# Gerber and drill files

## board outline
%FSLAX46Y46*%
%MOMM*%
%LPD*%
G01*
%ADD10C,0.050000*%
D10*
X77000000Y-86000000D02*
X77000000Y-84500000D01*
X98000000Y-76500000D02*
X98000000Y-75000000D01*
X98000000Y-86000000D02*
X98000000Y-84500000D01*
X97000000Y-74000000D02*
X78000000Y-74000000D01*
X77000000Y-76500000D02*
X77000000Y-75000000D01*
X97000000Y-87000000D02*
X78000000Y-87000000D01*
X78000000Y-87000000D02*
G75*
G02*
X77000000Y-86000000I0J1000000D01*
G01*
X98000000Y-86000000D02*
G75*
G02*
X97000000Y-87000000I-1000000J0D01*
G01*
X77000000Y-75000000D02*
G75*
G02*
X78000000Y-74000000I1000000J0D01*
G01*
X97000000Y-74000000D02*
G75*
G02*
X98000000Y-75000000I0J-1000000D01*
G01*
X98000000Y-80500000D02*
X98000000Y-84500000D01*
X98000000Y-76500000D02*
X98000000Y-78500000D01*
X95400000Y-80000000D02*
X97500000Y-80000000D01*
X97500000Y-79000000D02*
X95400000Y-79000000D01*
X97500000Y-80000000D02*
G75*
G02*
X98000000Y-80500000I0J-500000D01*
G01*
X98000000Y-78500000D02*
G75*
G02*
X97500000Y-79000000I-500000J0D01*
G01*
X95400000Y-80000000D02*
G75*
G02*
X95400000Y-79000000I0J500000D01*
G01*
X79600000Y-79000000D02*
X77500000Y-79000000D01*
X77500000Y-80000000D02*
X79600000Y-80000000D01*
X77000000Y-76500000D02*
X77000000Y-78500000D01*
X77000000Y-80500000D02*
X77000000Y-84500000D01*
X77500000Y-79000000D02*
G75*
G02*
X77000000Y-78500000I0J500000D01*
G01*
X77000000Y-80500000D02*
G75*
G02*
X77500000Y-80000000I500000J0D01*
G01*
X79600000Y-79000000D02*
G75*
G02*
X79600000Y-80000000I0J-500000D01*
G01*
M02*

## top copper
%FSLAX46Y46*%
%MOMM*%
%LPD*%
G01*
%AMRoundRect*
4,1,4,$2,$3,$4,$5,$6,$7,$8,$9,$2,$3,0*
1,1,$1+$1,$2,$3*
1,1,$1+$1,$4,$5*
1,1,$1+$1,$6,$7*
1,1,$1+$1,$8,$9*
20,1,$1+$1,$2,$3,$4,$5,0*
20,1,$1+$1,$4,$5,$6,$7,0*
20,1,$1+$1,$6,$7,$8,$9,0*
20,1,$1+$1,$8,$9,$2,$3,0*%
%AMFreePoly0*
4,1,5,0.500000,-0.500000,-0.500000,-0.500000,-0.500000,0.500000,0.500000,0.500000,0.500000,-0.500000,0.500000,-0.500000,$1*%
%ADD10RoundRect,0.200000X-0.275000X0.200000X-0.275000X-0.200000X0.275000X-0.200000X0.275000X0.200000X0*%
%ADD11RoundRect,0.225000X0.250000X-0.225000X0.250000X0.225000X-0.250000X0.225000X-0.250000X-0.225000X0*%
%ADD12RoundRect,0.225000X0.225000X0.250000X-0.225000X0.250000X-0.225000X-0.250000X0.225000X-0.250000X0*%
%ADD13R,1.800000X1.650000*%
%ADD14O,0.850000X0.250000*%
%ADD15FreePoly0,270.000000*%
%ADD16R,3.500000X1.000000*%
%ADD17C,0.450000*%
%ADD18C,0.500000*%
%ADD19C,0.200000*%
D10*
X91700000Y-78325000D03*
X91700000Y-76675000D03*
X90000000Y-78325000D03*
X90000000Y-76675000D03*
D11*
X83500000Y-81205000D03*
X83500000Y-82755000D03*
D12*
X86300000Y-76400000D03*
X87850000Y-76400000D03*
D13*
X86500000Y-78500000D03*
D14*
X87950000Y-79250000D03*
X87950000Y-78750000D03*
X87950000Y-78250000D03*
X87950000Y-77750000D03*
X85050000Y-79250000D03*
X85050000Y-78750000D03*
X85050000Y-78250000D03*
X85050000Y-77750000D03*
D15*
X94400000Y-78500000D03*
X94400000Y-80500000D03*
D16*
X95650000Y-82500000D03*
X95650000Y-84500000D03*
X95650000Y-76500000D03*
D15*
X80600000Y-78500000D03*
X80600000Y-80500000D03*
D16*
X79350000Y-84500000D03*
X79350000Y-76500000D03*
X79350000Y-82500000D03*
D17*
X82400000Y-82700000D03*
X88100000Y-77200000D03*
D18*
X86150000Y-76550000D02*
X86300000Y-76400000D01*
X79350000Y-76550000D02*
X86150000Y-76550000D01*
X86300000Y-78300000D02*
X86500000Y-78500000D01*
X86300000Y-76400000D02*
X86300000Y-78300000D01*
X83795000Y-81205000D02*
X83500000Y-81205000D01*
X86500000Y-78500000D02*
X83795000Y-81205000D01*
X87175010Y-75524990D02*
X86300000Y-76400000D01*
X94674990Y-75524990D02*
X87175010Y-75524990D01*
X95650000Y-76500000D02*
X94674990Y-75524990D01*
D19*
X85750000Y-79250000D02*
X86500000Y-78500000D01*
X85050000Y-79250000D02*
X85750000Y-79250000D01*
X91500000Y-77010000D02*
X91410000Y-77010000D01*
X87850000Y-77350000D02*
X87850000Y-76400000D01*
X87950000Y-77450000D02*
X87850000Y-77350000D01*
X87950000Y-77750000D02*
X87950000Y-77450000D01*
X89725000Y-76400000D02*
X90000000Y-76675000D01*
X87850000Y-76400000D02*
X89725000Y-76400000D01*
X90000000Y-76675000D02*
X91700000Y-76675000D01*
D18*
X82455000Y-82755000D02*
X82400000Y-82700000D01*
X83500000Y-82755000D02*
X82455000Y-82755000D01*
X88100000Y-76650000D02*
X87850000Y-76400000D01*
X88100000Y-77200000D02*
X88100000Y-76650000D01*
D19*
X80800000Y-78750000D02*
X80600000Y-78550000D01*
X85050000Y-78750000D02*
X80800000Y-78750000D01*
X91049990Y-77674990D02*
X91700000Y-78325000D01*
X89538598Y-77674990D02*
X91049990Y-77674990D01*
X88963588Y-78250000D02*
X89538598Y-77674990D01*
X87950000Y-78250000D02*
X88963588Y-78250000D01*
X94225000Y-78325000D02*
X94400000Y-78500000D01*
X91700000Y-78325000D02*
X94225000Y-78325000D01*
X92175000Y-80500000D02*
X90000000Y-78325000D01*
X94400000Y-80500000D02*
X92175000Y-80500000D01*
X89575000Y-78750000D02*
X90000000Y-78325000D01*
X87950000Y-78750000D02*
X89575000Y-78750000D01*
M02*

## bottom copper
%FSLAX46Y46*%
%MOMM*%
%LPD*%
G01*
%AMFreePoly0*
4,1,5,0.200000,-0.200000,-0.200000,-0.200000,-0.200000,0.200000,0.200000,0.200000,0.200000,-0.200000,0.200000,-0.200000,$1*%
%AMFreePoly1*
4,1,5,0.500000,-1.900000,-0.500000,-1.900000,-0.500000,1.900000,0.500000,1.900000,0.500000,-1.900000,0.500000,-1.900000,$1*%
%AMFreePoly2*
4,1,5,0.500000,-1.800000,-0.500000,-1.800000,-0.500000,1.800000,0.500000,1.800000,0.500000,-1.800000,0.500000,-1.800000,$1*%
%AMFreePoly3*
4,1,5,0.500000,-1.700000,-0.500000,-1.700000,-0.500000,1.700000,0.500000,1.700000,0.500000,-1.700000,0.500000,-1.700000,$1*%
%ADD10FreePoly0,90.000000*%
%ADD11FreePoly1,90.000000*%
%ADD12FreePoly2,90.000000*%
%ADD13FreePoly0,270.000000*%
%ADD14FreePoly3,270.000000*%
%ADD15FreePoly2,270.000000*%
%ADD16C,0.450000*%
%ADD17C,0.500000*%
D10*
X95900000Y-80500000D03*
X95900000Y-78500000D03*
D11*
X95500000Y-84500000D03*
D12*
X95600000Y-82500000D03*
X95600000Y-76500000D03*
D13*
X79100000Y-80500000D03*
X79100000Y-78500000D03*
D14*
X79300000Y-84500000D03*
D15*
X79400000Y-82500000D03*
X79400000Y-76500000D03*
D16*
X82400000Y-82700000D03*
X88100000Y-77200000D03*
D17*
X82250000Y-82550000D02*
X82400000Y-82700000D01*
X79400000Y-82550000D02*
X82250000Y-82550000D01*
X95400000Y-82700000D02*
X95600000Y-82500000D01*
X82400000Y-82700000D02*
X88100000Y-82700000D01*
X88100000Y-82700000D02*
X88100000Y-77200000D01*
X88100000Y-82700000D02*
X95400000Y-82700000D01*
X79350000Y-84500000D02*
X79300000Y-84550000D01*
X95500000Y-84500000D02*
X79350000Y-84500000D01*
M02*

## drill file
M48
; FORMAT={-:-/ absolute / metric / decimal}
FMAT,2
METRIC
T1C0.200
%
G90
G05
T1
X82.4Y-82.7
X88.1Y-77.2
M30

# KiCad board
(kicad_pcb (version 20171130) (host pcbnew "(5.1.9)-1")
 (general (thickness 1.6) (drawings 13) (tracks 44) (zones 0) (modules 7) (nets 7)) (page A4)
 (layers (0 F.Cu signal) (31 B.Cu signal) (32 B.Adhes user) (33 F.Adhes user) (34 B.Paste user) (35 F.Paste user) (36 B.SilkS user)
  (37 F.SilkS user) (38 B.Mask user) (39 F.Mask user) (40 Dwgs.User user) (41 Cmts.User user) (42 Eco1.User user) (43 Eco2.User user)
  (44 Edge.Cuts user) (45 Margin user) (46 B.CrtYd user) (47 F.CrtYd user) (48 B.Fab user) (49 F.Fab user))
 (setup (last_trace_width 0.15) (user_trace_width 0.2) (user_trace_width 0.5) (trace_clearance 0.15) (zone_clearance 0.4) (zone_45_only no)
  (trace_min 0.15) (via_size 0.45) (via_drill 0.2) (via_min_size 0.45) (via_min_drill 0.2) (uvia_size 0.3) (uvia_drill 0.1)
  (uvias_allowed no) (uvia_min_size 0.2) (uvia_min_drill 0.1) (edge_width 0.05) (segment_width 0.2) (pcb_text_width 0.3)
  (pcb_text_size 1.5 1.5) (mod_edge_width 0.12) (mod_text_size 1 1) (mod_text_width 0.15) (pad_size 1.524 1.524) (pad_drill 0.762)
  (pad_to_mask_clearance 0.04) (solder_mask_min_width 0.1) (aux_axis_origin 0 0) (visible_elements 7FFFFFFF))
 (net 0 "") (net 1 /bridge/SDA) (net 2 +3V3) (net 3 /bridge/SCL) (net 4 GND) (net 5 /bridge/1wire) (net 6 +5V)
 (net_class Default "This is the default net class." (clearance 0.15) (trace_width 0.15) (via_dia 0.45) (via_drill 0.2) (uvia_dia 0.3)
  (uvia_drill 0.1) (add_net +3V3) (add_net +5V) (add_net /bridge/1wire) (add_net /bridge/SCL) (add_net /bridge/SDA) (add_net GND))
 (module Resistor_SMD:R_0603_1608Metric (layer F.Cu) (at 91.7 77.5 270)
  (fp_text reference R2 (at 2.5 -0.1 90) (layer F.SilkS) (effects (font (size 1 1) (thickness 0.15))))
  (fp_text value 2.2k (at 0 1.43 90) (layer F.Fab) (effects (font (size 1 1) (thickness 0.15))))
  (pad 2 smd roundrect (at 0.825 0 270) (size 0.8 0.95) (layers F.Cu F.Paste F.Mask) (roundrect_rratio 0.25) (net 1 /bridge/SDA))
  (pad 1 smd roundrect (at -0.825 0 270) (size 0.8 0.95) (layers F.Cu F.Paste F.Mask) (roundrect_rratio 0.25) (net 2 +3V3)))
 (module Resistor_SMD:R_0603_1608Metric (layer F.Cu) (at 90 77.5 270)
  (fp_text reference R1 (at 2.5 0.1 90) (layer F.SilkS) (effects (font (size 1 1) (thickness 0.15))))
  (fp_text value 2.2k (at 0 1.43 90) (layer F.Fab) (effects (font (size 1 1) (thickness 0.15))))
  (pad 2 smd roundrect (at 0.825 0 270) (size 0.8 0.95) (layers F.Cu F.Paste F.Mask) (roundrect_rratio 0.25) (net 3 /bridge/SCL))
  (pad 1 smd roundrect (at -0.825 0 270) (size 0.8 0.95) (layers F.Cu F.Paste F.Mask) (roundrect_rratio 0.25) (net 2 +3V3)))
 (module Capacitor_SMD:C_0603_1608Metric (layer F.Cu) (at 83.5 81.98 90)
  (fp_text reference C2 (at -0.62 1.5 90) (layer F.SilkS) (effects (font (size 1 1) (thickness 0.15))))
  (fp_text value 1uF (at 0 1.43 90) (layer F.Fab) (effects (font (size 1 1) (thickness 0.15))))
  (pad 2 smd roundrect (at 0.775 0 90) (size 0.9 0.95) (layers F.Cu F.Paste F.Mask) (roundrect_rratio 0.25) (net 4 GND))
  (pad 1 smd roundrect (at -0.775 0 90) (size 0.9 0.95) (layers F.Cu F.Paste F.Mask) (roundrect_rratio 0.25) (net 2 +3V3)))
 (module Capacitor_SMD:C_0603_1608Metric (layer F.Cu) (at 87.075 76.4 180)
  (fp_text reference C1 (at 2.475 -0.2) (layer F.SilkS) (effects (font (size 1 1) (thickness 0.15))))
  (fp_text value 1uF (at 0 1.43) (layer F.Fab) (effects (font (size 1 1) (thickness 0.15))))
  (pad 2 smd roundrect (at 0.775 0 180) (size 0.9 0.95) (layers F.Cu F.Paste F.Mask) (roundrect_rratio 0.25) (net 4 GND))
  (pad 1 smd roundrect (at -0.775 0 180) (size 0.9 0.95) (layers F.Cu F.Paste F.Mask) (roundrect_rratio 0.25) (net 2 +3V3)))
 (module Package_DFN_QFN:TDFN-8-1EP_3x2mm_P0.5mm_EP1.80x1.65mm (layer F.Cu) (at 86.5 78.5)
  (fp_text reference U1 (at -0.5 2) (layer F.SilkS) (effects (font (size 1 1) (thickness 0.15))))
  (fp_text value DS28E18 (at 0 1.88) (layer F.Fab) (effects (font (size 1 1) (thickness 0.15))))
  (pad "" smd rect (at 0 0.5) (size 0.7 0.65) (layers F.Paste))
  (pad "" smd rect (at 0 -0.5) (size 0.7 0.65) (layers F.Paste)) (pad "" smd rect (at 0 0) (size 1.8 0.7) (layers F.Paste))
  (pad 9 smd rect (at 0 0) (size 1.8 1.65) (layers F.Cu F.Mask) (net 4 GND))
  (pad 5 smd oval (at 1.45 0.75) (size 0.85 0.25) (layers F.Cu F.Paste F.Mask))
  (pad 6 smd oval (at 1.45 0.25) (size 0.85 0.25) (layers F.Cu F.Paste F.Mask) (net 3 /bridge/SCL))
  (pad 7 smd oval (at 1.45 -0.25) (size 0.85 0.25) (layers F.Cu F.Paste F.Mask) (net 1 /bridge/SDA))
  (pad 8 smd oval (at 1.45 -0.75) (size 0.85 0.25) (layers F.Cu F.Paste F.Mask) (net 2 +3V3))
  (pad 4 smd oval (at -1.45 0.75) (size 0.85 0.25) (layers F.Cu F.Paste F.Mask) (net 4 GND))
  (pad 3 smd oval (at -1.45 0.25) (size 0.85 0.25) (layers F.Cu F.Paste F.Mask) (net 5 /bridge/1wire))
  (pad 2 smd oval (at -1.45 -0.25) (size 0.85 0.25) (layers F.Cu F.Paste F.Mask))
  (pad 1 smd oval (at -1.45 -0.75) (size 0.85 0.25) (layers F.Cu F.Paste F.Mask)))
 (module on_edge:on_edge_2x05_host (layer F.Cu) (at 98 80.5 270)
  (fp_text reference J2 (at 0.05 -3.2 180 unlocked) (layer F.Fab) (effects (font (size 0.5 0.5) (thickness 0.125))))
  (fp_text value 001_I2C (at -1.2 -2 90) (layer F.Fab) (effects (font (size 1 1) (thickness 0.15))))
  (fp_line (start 0 0) (end 4 0) (layer Edge.Cuts) (width 0.05))
  (fp_line (start -4 0) (end -2 0) (layer Edge.Cuts) (width 0.05))
  (fp_line (start -0.5 2.6) (end -0.5 0.5) (layer Edge.Cuts) (width 0.05))
  (fp_line (start -1.5 0.5) (end -1.5 2.6) (layer Edge.Cuts) (width 0.05))
  (fp_arc (start 0 0.5) (end 0 0) (angle -90) (layer Edge.Cuts) (width 0.05))
  (fp_arc (start -2 0.5) (end -1.5 0.5) (angle -90) (layer Edge.Cuts) (width 0.05))
  (fp_arc (start -1 2.6) (end -1.5 2.6) (angle -180) (layer Edge.Cuts) (width 0.05))
  (pad 2 smd custom (at -2 3.6 270) (size 1 1) (layers F.Cu F.Mask) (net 1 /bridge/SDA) (zone_connect 0)
   (options (clearance outline) (anchor rect)) (primitives))
  (pad 3 smd custom (at 0 3.6 270) (size 1 1) (layers F.Cu F.Mask) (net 3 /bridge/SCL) (zone_connect 0)
   (options (clearance outline) (anchor rect)) (primitives))
  (pad 8 smd custom (at 0 2.1 90) (size 0.4 0.4) (layers B.Cu B.Mask) (zone_connect 0) (options (clearance outline) (anchor rect))
   (primitives))
  (pad 7 smd custom (at -2 2.1 90) (size 0.4 0.4) (layers B.Cu B.Mask) (zone_connect 0) (options (clearance outline) (anchor rect))
   (primitives))
  (pad 4 smd rect (at 2 2.35 270) (size 1 3.5) (layers F.Cu F.Mask) (zone_connect 0))
  (pad 10 smd custom (at 4 2.5 90) (size 1 3.8) (layers B.Cu B.Mask) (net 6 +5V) (zone_connect 0)
   (options (clearance outline) (anchor rect)) (primitives))
  (pad 9 smd custom (at 2 2.4 90) (size 1 3.6) (layers B.Cu B.Mask) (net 2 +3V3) (zone_connect 0)
   (options (clearance outline) (anchor rect)) (primitives))
  (pad 6 smd custom (at -4 2.4 90) (size 1 3.6) (layers B.Cu B.Mask) (zone_connect 0) (options (clearance outline) (anchor rect))
   (primitives))
  (pad 5 smd rect (at 4 2.35 270) (size 1 3.5) (layers F.Cu F.Mask) (zone_connect 0))
  (pad 1 smd rect (at -4 2.35 270) (size 1 3.5) (layers F.Cu F.Mask) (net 4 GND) (zone_connect 0)))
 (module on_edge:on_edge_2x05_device (layer F.Cu) (at 77 80.5 270)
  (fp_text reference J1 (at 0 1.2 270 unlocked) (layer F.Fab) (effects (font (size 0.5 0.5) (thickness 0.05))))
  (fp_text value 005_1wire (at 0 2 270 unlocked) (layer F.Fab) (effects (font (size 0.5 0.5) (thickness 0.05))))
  (fp_line (start -1.5 -2.6) (end -1.5 -0.5) (layer Edge.Cuts) (width 0.05))
  (fp_line (start -0.5 -0.5) (end -0.5 -2.6) (layer Edge.Cuts) (width 0.05))
  (fp_line (start -4 0) (end -2 0) (layer Edge.Cuts) (width 0.05))
  (fp_line (start 0 0) (end 4 0) (layer Edge.Cuts) (width 0.05))
  (fp_arc (start -2 -0.5) (end -2 0) (angle -90) (layer Edge.Cuts) (width 0.05))
  (fp_arc (start 0 -0.5) (end -0.5 -0.5) (angle -90) (layer Edge.Cuts) (width 0.05))
  (fp_arc (start -1 -2.6) (end -0.5 -2.6) (angle -180) (layer Edge.Cuts) (width 0.05))
  (pad 2 smd custom (at -2 -3.6 270) (size 1 1) (layers F.Cu F.Mask) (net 5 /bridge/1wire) (zone_connect 0)
   (options (clearance outline) (anchor rect)) (primitives))
  (pad 3 smd custom (at 0 -3.6 270) (size 1 1) (layers F.Cu F.Mask) (zone_connect 0) (options (clearance outline) (anchor rect))
   (primitives))
  (pad 8 smd custom (at 0 -2.1 270) (size 0.4 0.4) (layers B.Cu B.Mask) (zone_connect 0) (options (clearance outline) (anchor rect))
   (primitives))
  (pad 7 smd custom (at -2 -2.1 270) (size 0.4 0.4) (layers B.Cu B.Mask) (zone_connect 0) (options (clearance outline) (anchor rect))
   (primitives))
  (pad 10 smd custom (at 4 -2.3 270) (size 1 3.4) (layers B.Cu B.Mask) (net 6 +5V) (zone_connect 0)
   (options (clearance outline) (anchor rect)) (primitives))
  (pad 9 smd custom (at 2 -2.4 270) (size 1 3.6) (layers B.Cu B.Mask) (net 2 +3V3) (zone_connect 0)
   (options (clearance outline) (anchor rect)) (primitives))
  (pad 6 smd custom (at -4 -2.4 270) (size 1 3.6) (layers B.Cu B.Mask) (zone_connect 0) (options (clearance outline) (anchor rect))
   (primitives))
  (pad 5 smd rect (at 4 -2.35 90) (size 1 3.5) (layers F.Cu F.Mask) (zone_connect 0))
  (pad 1 smd rect (at -4 -2.35 90) (size 1 3.5) (layers F.Cu F.Mask) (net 4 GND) (zone_connect 0))
  (pad 4 smd rect (at 2 -2.35 90) (size 1 3.5) (layers F.Cu F.Mask) (zone_connect 0)))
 (gr_line (start 77 86) (end 77 84.5) (layer Edge.Cuts) (width 0.05))
 (gr_line (start 98 76.5) (end 98 75) (layer Edge.Cuts) (width 0.05))
 (gr_line (start 98 86) (end 98 84.5) (layer Edge.Cuts) (width 0.05))
 (gr_line (start 97 74) (end 78 74) (layer Edge.Cuts) (width 0.05))
 (gr_line (start 77 76.5) (end 77 75) (layer Edge.Cuts) (width 0.05))
 (gr_line (start 97 87) (end 78 87) (layer Edge.Cuts) (width 0.05))
 (gr_arc (start 78 86) (end 77 86) (angle -90) (layer Edge.Cuts) (width 0.05))
 (gr_arc (start 97 86) (end 97 87) (angle -90) (layer Edge.Cuts) (width 0.05))
 (gr_arc (start 78 75) (end 78 74) (angle -90) (layer Edge.Cuts) (width 0.05))
 (gr_arc (start 97 75) (end 98 75) (angle -90) (layer Edge.Cuts) (width 0.05))
 (segment (start 86.15 76.55) (end 86.3 76.4) (width 0.5) (layer F.Cu) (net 4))
 (segment (start 79.35 76.55) (end 86.15 76.55) (width 0.5) (layer F.Cu) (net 4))
 (segment (start 86.3 78.3) (end 86.5 78.5) (width 0.5) (layer F.Cu) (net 4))
 (segment (start 86.3 76.4) (end 86.3 78.3) (width 0.5) (layer F.Cu) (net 4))
 (segment (start 83.795 81.205) (end 83.5 81.205) (width 0.5) (layer F.Cu) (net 4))
 (segment (start 86.5 78.5) (end 83.795 81.205) (width 0.5) (layer F.Cu) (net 4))
 (segment (start 87.17501 75.52499) (end 86.3 76.4) (width 0.5) (layer F.Cu) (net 4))
 (segment (start 94.67499 75.52499) (end 87.17501 75.52499) (width 0.5) (layer F.Cu) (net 4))
 (segment (start 95.65 76.5) (end 94.67499 75.52499) (width 0.5) (layer F.Cu) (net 4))
 (segment (start 85.75 79.25) (end 86.5 78.5) (width 0.2) (layer F.Cu) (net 4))
 (segment (start 85.05 79.25) (end 85.75 79.25) (width 0.2) (layer F.Cu) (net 4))
 (segment (start 82.25 82.55) (end 82.4 82.7) (width 0.5) (layer B.Cu) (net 2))
 (via (at 82.4 82.7) (size 0.45) (drill 0.2) (layers F.Cu B.Cu) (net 2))
 (segment (start 79.4 82.55) (end 82.25 82.55) (width 0.5) (layer B.Cu) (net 2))
 (segment (start 91.5 77.01) (end 91.41 77.01) (width 0.2) (layer F.Cu) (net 2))
 (segment (start 87.85 77.35) (end 87.85 76.4) (width 0.2) (layer F.Cu) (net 2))
 (segment (start 87.95 77.45) (end 87.85 77.35) (width 0.2) (layer F.Cu) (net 2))
 (segment (start 87.95 77.75) (end 87.95 77.45) (width 0.2) (layer F.Cu) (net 2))
 (segment (start 89.725 76.4) (end 90 76.675) (width 0.2) (layer F.Cu) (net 2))
 (segment (start 87.85 76.4) (end 89.725 76.4) (width 0.2) (layer F.Cu) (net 2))
 (segment (start 90 76.675) (end 91.7 76.675) (width 0.2) (layer F.Cu) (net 2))
 (segment (start 82.455 82.755) (end 82.4 82.7) (width 0.5) (layer F.Cu) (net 2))
 (segment (start 83.5 82.755) (end 82.455 82.755) (width 0.5) (layer F.Cu) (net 2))
 (segment (start 95.4 82.7) (end 95.6 82.5) (width 0.5) (layer B.Cu) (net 2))
 (via (at 88.1 77.2) (size 0.45) (drill 0.2) (layers F.Cu B.Cu) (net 2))
 (segment (start 82.4 82.7) (end 88.1 82.7) (width 0.5) (layer B.Cu) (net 2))
 (segment (start 88.1 82.7) (end 88.1 77.2) (width 0.5) (layer B.Cu) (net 2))
 (segment (start 88.1 82.7) (end 95.4 82.7) (width 0.5) (layer B.Cu) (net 2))
 (segment (start 88.1 76.65) (end 87.85 76.4) (width 0.5) (layer F.Cu) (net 2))
 (segment (start 88.1 77.2) (end 88.1 76.65) (width 0.5) (layer F.Cu) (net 2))
 (segment (start 80.8 78.75) (end 80.6 78.55) (width 0.2) (layer F.Cu) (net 5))
 (segment (start 85.05 78.75) (end 80.8 78.75) (width 0.2) (layer F.Cu) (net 5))
 (segment (start 79.35 84.5) (end 79.3 84.55) (width 0.5) (layer B.Cu) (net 6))
 (segment (start 95.5 84.5) (end 79.35 84.5) (width 0.5) (layer B.Cu) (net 6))
 (segment (start 91.04999 77.67499) (end 91.7 78.325) (width 0.2) (layer F.Cu) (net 1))
 (segment (start 89.538598 77.67499) (end 91.04999 77.67499) (width 0.2) (layer F.Cu) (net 1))
 (segment (start 88.963588 78.25) (end 89.538598 77.67499) (width 0.2) (layer F.Cu) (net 1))
 (segment (start 87.95 78.25) (end 88.963588 78.25) (width 0.2) (layer F.Cu) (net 1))
 (segment (start 94.225 78.325) (end 94.4 78.5) (width 0.2) (layer F.Cu) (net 1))
 (segment (start 91.7 78.325) (end 94.225 78.325) (width 0.2) (layer F.Cu) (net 1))
 (segment (start 92.175 80.5) (end 90 78.325) (width 0.2) (layer F.Cu) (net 3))
 (segment (start 94.4 80.5) (end 92.175 80.5) (width 0.2) (layer F.Cu) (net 3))
 (segment (start 89.575 78.75) (end 90 78.325) (width 0.2) (layer F.Cu) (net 3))
 (segment (start 87.95 78.75) (end 89.575 78.75) (width 0.2) (layer F.Cu) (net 3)))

